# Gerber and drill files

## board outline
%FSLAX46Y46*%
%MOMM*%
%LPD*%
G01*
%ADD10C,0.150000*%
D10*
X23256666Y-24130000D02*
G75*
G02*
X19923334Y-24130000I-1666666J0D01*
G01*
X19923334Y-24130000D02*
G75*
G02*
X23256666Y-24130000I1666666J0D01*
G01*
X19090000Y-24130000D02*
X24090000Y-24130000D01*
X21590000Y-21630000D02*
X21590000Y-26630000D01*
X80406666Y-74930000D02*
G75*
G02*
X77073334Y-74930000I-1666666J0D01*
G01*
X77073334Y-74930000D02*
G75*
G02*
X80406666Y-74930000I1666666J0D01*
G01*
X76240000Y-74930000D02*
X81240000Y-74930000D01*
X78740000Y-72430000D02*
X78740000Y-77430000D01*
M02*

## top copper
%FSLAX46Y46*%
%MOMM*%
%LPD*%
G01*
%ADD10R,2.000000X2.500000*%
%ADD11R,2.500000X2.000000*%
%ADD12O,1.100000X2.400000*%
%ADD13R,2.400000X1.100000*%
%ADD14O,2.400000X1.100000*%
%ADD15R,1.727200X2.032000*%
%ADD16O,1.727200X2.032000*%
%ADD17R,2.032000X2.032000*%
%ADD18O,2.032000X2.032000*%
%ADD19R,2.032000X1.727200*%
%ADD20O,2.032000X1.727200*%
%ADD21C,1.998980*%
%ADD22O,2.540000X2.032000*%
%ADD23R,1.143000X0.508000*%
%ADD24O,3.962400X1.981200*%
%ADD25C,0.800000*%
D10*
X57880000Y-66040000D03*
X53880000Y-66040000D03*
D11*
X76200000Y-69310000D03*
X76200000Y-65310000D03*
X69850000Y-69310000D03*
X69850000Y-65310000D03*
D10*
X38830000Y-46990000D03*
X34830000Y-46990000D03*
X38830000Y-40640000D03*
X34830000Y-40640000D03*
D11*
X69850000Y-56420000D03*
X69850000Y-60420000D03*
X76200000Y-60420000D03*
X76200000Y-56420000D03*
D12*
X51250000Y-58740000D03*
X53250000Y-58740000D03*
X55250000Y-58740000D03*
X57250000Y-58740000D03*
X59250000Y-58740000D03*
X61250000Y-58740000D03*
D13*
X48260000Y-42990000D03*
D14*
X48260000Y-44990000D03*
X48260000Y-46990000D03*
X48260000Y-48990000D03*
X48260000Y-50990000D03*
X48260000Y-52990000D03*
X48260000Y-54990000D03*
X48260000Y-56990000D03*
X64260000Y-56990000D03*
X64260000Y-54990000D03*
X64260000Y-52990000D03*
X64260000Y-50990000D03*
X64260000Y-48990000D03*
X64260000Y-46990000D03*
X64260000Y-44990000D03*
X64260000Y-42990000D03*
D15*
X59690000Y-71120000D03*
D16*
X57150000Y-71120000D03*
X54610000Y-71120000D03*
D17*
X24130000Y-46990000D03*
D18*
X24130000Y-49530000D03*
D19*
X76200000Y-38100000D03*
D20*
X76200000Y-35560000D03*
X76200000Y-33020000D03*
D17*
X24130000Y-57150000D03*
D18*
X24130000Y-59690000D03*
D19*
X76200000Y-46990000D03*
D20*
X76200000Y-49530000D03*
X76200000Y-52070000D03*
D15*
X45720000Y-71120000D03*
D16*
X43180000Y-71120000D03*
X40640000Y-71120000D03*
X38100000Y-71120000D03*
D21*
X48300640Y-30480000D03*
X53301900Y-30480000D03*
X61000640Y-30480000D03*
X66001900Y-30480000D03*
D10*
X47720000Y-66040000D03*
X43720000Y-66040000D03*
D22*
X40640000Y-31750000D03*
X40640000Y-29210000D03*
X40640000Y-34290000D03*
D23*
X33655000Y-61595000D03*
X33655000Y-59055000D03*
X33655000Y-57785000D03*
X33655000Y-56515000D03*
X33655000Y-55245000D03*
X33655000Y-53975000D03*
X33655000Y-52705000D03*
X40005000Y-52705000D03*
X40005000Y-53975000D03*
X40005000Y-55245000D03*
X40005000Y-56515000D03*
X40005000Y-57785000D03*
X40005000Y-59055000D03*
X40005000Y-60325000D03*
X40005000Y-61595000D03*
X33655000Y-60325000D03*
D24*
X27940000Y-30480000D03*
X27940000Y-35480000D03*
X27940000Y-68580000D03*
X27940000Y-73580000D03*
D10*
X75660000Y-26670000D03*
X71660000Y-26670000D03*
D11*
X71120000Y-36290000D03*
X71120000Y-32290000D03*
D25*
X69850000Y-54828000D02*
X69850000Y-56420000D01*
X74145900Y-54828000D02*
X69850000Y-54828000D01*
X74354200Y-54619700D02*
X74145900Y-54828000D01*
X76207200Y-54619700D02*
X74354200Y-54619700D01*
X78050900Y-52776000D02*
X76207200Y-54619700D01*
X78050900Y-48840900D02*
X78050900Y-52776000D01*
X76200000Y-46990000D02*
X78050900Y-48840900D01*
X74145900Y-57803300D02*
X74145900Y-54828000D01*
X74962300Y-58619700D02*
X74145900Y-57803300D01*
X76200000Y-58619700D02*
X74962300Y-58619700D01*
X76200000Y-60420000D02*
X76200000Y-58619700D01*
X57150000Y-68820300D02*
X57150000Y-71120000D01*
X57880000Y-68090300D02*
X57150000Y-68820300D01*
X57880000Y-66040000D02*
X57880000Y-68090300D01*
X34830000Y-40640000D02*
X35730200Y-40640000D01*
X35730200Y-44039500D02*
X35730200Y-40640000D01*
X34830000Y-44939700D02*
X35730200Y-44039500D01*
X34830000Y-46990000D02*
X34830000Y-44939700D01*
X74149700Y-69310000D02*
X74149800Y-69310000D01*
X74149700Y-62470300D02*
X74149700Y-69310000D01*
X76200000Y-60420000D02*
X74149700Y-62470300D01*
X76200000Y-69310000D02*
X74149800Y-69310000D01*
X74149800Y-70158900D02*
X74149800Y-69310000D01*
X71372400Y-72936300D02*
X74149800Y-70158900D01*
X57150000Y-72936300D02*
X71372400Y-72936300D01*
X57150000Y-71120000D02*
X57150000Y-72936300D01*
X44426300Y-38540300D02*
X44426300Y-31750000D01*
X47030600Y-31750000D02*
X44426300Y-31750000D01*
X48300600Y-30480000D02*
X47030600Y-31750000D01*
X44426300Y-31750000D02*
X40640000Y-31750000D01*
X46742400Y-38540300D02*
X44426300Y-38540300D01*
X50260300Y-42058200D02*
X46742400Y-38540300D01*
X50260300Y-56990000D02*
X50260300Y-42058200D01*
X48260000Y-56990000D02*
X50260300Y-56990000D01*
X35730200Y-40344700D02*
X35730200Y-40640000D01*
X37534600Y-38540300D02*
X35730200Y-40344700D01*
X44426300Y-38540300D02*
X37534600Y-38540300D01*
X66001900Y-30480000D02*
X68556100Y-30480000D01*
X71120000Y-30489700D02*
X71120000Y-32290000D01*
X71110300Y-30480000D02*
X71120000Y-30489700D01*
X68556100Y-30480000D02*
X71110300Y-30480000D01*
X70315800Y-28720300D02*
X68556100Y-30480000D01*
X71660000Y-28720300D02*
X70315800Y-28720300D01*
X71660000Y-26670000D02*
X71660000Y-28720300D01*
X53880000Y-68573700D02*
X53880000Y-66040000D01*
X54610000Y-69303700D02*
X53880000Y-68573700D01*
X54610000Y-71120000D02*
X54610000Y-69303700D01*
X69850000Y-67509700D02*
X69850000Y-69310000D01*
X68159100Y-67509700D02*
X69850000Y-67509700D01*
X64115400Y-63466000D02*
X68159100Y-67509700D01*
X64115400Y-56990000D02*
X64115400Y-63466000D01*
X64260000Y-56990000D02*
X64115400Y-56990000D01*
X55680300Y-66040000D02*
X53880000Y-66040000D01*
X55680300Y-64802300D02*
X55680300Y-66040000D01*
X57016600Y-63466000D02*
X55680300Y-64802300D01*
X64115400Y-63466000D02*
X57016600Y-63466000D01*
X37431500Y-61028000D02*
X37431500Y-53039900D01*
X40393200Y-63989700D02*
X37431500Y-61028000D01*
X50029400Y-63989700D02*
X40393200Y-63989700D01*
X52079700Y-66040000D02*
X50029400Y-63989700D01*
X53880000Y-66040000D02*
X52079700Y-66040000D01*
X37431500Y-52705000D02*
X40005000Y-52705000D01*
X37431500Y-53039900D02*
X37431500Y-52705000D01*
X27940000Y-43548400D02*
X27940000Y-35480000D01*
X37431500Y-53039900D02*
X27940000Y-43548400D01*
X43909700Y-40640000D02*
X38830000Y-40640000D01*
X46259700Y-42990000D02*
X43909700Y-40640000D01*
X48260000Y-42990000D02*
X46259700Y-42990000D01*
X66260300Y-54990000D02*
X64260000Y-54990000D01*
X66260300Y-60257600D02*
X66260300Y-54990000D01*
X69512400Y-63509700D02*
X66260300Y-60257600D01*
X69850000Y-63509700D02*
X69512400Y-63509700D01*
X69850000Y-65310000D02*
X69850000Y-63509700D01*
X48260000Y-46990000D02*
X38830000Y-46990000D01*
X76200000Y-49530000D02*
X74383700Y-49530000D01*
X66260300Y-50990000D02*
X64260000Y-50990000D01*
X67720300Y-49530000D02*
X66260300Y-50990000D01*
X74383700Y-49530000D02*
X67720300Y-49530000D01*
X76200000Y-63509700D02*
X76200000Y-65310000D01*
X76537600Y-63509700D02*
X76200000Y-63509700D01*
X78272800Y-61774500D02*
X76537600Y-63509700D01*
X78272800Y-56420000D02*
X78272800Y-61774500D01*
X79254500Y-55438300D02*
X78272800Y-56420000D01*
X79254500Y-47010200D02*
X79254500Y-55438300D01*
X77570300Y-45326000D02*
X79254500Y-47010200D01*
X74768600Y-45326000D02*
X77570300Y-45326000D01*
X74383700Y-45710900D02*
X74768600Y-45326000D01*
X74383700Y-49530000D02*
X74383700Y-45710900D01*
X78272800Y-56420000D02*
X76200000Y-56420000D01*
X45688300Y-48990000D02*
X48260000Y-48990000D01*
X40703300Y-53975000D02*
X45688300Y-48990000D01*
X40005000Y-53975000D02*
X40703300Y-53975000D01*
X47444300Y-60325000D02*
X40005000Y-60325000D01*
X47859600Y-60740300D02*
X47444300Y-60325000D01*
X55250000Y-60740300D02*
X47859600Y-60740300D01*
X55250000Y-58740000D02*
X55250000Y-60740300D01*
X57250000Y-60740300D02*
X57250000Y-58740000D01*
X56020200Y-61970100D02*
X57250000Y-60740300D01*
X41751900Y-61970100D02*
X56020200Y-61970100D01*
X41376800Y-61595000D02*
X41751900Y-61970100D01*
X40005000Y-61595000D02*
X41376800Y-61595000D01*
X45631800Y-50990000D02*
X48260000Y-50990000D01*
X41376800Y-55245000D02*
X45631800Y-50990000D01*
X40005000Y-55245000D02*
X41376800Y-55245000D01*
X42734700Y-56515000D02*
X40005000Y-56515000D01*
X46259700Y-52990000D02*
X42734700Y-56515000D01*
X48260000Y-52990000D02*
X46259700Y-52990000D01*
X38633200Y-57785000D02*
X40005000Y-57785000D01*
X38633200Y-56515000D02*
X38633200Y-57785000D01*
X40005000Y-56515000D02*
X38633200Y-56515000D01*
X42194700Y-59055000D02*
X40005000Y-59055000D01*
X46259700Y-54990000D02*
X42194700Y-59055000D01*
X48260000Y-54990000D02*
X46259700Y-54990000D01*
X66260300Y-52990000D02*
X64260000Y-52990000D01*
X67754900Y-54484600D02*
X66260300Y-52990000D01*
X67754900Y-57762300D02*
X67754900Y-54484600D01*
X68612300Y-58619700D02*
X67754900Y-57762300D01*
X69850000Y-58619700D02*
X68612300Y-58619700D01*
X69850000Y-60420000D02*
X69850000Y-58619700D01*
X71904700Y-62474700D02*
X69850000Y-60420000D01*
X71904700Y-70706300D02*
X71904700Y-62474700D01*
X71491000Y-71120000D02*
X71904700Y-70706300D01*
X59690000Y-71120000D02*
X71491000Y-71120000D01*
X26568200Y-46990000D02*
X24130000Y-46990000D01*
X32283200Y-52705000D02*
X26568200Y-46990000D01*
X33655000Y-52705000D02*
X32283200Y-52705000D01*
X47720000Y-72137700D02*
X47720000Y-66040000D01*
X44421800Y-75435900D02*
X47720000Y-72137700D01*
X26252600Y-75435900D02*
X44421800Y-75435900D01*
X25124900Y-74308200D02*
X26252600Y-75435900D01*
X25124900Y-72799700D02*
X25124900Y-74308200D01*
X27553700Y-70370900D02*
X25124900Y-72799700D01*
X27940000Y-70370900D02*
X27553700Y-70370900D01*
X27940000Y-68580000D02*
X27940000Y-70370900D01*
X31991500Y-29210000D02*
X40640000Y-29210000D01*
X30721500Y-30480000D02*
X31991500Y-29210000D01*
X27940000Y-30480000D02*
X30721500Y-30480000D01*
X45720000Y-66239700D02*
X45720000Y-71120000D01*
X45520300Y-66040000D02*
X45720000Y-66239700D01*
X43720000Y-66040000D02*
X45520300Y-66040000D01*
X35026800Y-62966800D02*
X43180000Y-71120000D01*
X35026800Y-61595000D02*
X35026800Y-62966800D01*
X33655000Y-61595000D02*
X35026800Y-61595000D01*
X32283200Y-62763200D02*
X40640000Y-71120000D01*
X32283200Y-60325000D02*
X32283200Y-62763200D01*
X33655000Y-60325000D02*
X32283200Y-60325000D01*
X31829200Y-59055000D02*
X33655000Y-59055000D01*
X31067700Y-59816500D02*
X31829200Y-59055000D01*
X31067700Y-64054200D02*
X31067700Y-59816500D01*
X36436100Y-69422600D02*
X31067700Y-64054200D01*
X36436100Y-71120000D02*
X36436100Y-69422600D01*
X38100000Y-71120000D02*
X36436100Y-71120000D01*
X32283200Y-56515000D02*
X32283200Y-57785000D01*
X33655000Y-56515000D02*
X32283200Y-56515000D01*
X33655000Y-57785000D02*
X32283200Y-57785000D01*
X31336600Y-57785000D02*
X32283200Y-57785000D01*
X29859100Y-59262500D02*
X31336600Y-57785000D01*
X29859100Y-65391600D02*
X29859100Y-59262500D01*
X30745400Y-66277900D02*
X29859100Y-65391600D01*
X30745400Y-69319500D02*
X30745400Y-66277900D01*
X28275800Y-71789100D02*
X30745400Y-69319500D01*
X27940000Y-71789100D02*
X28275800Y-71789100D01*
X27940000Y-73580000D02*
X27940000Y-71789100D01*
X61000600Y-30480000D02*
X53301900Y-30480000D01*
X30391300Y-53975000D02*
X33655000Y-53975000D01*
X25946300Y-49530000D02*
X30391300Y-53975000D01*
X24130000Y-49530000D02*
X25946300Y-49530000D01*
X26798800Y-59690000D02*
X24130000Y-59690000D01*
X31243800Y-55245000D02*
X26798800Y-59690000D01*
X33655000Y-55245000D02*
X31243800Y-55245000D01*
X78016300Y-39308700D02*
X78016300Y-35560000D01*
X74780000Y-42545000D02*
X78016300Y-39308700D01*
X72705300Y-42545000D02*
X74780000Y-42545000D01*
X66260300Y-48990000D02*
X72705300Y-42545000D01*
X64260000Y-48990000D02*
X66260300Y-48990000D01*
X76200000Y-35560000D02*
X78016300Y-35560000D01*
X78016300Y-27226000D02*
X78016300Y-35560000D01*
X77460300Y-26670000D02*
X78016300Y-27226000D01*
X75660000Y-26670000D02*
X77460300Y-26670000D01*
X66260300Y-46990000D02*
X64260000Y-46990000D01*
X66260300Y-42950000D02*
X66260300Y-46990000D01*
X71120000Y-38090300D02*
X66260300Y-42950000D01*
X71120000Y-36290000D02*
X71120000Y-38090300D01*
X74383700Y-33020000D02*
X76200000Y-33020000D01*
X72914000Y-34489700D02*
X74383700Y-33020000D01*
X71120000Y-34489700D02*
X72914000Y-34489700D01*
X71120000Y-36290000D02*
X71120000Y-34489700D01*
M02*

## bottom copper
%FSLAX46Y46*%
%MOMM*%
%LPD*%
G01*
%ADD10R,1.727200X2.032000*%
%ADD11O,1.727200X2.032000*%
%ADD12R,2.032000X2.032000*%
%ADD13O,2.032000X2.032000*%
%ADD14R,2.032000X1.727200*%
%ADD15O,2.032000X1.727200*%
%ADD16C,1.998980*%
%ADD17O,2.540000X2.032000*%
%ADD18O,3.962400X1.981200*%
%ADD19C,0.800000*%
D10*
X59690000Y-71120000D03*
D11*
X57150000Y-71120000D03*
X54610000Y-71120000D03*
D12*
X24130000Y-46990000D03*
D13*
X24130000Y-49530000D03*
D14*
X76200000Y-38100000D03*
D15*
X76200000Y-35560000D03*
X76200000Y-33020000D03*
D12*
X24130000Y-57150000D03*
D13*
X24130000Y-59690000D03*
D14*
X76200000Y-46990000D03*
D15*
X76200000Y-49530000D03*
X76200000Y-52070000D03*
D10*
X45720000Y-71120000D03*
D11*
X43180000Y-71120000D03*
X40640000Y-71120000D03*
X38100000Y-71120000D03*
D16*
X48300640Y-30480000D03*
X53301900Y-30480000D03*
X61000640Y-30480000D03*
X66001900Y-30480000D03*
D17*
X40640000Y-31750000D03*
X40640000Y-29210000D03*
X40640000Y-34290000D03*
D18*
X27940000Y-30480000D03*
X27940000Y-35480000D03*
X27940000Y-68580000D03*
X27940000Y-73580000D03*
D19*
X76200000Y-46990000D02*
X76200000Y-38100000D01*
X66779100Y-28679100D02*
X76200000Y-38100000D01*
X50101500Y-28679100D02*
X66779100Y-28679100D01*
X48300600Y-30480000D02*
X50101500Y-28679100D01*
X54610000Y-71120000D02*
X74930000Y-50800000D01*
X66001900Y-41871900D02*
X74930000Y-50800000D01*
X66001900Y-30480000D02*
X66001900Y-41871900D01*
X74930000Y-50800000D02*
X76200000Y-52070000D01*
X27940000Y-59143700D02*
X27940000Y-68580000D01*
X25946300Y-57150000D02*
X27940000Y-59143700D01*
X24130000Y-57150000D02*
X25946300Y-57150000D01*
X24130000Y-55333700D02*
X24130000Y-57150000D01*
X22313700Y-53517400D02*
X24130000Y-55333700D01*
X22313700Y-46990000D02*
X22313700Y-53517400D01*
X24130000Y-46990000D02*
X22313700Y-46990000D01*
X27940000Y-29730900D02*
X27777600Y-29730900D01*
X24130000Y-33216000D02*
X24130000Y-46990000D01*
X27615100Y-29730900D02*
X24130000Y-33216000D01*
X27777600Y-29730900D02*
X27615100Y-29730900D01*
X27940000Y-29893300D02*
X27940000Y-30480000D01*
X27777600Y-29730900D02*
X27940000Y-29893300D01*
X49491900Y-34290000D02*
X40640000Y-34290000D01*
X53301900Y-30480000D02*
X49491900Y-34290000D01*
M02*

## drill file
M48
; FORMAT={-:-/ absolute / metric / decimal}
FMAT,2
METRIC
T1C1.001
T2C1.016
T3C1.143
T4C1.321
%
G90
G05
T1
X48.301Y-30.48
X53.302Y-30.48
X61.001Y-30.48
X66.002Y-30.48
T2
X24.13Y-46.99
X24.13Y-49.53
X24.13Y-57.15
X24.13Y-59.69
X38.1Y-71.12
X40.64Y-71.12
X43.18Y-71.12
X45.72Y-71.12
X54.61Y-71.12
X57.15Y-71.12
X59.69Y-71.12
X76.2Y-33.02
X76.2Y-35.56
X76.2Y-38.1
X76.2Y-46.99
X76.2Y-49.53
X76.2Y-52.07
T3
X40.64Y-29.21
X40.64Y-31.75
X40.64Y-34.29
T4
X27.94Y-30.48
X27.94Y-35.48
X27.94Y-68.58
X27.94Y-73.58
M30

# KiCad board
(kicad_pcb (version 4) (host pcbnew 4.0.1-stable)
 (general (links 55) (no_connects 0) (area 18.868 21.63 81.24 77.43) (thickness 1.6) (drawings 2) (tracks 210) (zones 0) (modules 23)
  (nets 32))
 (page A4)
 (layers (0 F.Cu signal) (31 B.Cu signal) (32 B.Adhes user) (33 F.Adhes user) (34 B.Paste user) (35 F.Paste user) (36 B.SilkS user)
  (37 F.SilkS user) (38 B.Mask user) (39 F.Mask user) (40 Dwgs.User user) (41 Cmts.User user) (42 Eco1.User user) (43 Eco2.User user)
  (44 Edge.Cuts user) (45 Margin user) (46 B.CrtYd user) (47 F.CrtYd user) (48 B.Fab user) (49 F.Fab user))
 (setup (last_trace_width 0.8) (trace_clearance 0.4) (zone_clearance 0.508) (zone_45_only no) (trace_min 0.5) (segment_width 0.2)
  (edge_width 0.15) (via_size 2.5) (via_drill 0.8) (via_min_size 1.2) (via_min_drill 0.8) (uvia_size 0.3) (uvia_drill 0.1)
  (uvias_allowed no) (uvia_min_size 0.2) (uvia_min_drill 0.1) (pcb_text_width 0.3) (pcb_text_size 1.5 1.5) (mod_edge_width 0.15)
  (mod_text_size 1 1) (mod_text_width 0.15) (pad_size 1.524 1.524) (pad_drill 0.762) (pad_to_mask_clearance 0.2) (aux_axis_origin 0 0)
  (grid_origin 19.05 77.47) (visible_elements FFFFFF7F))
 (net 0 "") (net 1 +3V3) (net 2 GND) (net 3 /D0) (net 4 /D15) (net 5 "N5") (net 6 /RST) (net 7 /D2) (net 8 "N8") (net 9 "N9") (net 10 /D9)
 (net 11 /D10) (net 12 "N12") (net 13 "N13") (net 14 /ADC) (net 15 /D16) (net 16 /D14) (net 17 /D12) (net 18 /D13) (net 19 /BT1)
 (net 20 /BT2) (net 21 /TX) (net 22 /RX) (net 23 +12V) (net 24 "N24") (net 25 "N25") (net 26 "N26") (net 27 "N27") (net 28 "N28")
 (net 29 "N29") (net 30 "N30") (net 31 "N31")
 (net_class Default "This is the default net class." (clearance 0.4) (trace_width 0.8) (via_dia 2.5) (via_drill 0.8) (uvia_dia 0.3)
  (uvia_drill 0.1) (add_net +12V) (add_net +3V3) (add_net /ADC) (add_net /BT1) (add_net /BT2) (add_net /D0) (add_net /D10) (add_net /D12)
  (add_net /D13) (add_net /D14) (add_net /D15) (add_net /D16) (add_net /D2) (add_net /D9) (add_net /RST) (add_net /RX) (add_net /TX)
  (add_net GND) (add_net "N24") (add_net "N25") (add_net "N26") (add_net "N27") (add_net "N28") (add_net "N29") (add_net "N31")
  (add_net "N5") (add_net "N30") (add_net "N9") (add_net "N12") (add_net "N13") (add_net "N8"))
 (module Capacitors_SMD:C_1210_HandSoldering (layer F.Cu) (at 55.88 66.04 180)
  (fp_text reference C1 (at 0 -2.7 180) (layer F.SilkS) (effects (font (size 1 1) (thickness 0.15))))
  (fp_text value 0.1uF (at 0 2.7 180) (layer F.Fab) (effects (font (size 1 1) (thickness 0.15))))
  (pad 1 smd rect (at -2 0 180) (size 2 2.5) (layers F.Cu F.Paste F.Mask) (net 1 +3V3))
  (pad 2 smd rect (at 2 0 180) (size 2 2.5) (layers F.Cu F.Paste F.Mask) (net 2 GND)))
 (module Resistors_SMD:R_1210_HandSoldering (layer F.Cu) (at 76.2 67.31 90)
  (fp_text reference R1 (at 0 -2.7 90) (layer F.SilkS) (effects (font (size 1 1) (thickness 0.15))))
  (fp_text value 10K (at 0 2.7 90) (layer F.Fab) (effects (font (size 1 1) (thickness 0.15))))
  (pad 1 smd rect (at -2 0 90) (size 2 2.5) (layers F.Cu F.Paste F.Mask) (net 1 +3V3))
  (pad 2 smd rect (at 2 0 90) (size 2 2.5) (layers F.Cu F.Paste F.Mask) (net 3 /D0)))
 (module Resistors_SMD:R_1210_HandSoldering (layer F.Cu) (at 69.85 67.31 90)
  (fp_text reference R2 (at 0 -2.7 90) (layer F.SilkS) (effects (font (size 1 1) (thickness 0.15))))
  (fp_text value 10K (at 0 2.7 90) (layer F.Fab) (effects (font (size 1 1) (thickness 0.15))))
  (pad 1 smd rect (at -2 0 90) (size 2 2.5) (layers F.Cu F.Paste F.Mask) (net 2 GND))
  (pad 2 smd rect (at 2 0 90) (size 2 2.5) (layers F.Cu F.Paste F.Mask) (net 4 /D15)))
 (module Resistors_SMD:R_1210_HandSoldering (layer F.Cu) (at 36.83 46.99 180)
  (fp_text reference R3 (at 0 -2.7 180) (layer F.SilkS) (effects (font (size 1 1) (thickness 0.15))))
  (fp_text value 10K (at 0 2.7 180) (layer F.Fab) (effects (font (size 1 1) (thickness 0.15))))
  (pad 1 smd rect (at -2 0 180) (size 2 2.5) (layers F.Cu F.Paste F.Mask) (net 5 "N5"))
  (pad 2 smd rect (at 2 0 180) (size 2 2.5) (layers F.Cu F.Paste F.Mask) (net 1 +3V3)))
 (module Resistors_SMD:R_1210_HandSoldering (layer F.Cu) (at 36.83 40.64 180)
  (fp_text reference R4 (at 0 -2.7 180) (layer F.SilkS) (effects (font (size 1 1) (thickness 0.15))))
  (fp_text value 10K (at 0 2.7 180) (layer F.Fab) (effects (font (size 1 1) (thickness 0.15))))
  (pad 1 smd rect (at -2 0 180) (size 2 2.5) (layers F.Cu F.Paste F.Mask) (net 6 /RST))
  (pad 2 smd rect (at 2 0 180) (size 2 2.5) (layers F.Cu F.Paste F.Mask) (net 1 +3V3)))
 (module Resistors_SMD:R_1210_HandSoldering (layer F.Cu) (at 69.85 58.42 270)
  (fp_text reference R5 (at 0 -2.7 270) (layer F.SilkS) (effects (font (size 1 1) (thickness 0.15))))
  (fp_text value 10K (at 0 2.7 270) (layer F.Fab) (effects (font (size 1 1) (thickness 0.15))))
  (pad 1 smd rect (at -2 0 270) (size 2 2.5) (layers F.Cu F.Paste F.Mask) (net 1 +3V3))
  (pad 2 smd rect (at 2 0 270) (size 2 2.5) (layers F.Cu F.Paste F.Mask) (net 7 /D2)))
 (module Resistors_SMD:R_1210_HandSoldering (layer F.Cu) (at 76.2 58.42 90)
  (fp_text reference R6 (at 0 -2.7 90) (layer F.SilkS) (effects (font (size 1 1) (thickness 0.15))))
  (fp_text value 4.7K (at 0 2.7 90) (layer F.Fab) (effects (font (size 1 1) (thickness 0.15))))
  (pad 1 smd rect (at -2 0 90) (size 2 2.5) (layers F.Cu F.Paste F.Mask) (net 1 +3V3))
  (pad 2 smd rect (at 2 0 90) (size 2 2.5) (layers F.Cu F.Paste F.Mask) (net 3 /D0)))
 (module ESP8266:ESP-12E (layer F.Cu) (at 48.26 42.99)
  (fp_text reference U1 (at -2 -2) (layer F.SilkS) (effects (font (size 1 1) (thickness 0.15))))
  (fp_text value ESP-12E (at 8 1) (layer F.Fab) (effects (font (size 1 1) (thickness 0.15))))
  (pad 9 smd oval (at 2.99 15.75 90) (size 2.4 1.1) (layers F.Cu F.Paste F.Mask) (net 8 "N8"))
  (pad 10 smd oval (at 4.99 15.75 90) (size 2.4 1.1) (layers F.Cu F.Paste F.Mask) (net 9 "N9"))
  (pad 11 smd oval (at 6.99 15.75 90) (size 2.4 1.1) (layers F.Cu F.Paste F.Mask) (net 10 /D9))
  (pad 12 smd oval (at 8.99 15.75 90) (size 2.4 1.1) (layers F.Cu F.Paste F.Mask) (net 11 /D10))
  (pad 13 smd oval (at 10.99 15.75 90) (size 2.4 1.1) (layers F.Cu F.Paste F.Mask) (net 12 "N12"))
  (pad 14 smd oval (at 12.99 15.75 90) (size 2.4 1.1) (layers F.Cu F.Paste F.Mask) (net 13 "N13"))
  (pad 1 smd rect (at 0 0) (size 2.4 1.1) (layers F.Cu F.Paste F.Mask) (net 6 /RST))
  (pad 2 smd oval (at 0 2) (size 2.4 1.1) (layers F.Cu F.Paste F.Mask) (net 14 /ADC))
  (pad 3 smd oval (at 0 4) (size 2.4 1.1) (layers F.Cu F.Paste F.Mask) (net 5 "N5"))
  (pad 4 smd oval (at 0 6) (size 2.4 1.1) (layers F.Cu F.Paste F.Mask) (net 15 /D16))
  (pad 5 smd oval (at 0 8) (size 2.4 1.1) (layers F.Cu F.Paste F.Mask) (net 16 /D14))
  (pad 6 smd oval (at 0 10) (size 2.4 1.1) (layers F.Cu F.Paste F.Mask) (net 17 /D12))
  (pad 7 smd oval (at 0 12) (size 2.4 1.1) (layers F.Cu F.Paste F.Mask) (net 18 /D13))
  (pad 8 smd oval (at 0 14) (size 2.4 1.1) (layers F.Cu F.Paste F.Mask) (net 1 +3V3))
  (pad 15 smd oval (at 16 14) (size 2.4 1.1) (layers F.Cu F.Paste F.Mask) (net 2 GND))
  (pad 16 smd oval (at 16 12) (size 2.4 1.1) (layers F.Cu F.Paste F.Mask) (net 4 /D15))
  (pad 17 smd oval (at 16 10) (size 2.4 1.1) (layers F.Cu F.Paste F.Mask) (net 7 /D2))
  (pad 18 smd oval (at 16 8) (size 2.4 1.1) (layers F.Cu F.Paste F.Mask) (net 3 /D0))
  (pad 19 smd oval (at 16 6) (size 2.4 1.1) (layers F.Cu F.Paste F.Mask) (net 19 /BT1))
  (pad 20 smd oval (at 16 4) (size 2.4 1.1) (layers F.Cu F.Paste F.Mask) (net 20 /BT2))
  (pad 21 smd oval (at 16 2) (size 2.4 1.1) (layers F.Cu F.Paste F.Mask) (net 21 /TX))
  (pad 22 smd oval (at 16 0) (size 2.4 1.1) (layers F.Cu F.Paste F.Mask) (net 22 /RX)))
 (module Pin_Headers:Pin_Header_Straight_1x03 (layer F.Cu) (at 59.69 71.12 270)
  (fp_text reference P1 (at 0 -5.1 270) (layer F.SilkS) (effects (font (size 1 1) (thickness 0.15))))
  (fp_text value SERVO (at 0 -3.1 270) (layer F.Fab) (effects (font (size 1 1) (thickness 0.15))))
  (pad 1 thru_hole rect (at 0 0 270) (size 2.032 1.7272) (drill 1.016) (layers *.Cu *.Mask F.SilkS) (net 7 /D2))
  (pad 2 thru_hole oval (at 0 2.54 270) (size 2.032 1.7272) (drill 1.016) (layers *.Cu *.Mask F.SilkS) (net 1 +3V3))
  (pad 3 thru_hole oval (at 0 5.08 270) (size 2.032 1.7272) (drill 1.016) (layers *.Cu *.Mask F.SilkS) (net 2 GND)))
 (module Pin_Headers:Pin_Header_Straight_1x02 (layer F.Cu) (at 24.13 46.99)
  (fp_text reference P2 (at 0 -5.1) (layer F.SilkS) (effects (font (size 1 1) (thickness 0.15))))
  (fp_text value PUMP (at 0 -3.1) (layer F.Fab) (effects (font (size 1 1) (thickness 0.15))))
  (pad 1 thru_hole rect (at 0 0) (size 2.032 2.032) (drill 1.016) (layers *.Cu *.Mask F.SilkS) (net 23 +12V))
  (pad 2 thru_hole oval (at 0 2.54) (size 2.032 2.032) (drill 1.016) (layers *.Cu *.Mask F.SilkS) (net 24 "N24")))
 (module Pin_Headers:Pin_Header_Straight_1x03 (layer F.Cu) (at 76.2 38.1 180)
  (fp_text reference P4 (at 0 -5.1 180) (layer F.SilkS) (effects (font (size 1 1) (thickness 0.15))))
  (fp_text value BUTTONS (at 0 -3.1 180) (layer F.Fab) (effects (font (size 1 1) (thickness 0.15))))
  (pad 1 thru_hole rect (at 0 0 180) (size 2.032 1.7272) (drill 1.016) (layers *.Cu *.Mask F.SilkS) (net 1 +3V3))
  (pad 2 thru_hole oval (at 0 2.54 180) (size 2.032 1.7272) (drill 1.016) (layers *.Cu *.Mask F.SilkS) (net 19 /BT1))
  (pad 3 thru_hole oval (at 0 5.08 180) (size 2.032 1.7272) (drill 1.016) (layers *.Cu *.Mask F.SilkS) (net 20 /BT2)))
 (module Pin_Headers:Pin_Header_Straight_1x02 (layer F.Cu) (at 24.13 57.15)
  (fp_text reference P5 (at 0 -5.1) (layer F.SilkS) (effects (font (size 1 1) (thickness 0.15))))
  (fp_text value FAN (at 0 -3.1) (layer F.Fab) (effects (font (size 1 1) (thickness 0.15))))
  (pad 1 thru_hole rect (at 0 0) (size 2.032 2.032) (drill 1.016) (layers *.Cu *.Mask F.SilkS) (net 23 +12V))
  (pad 2 thru_hole oval (at 0 2.54) (size 2.032 2.032) (drill 1.016) (layers *.Cu *.Mask F.SilkS) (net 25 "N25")))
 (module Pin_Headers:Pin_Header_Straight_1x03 (layer F.Cu) (at 76.2 46.99)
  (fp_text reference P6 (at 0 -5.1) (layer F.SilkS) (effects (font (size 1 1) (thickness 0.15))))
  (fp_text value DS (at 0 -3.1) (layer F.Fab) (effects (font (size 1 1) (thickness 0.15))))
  (pad 1 thru_hole rect (at 0 0) (size 2.032 1.7272) (drill 1.016) (layers *.Cu *.Mask F.SilkS) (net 1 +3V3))
  (pad 2 thru_hole oval (at 0 2.54) (size 2.032 1.7272) (drill 1.016) (layers *.Cu *.Mask F.SilkS) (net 3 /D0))
  (pad 3 thru_hole oval (at 0 5.08) (size 2.032 1.7272) (drill 1.016) (layers *.Cu *.Mask F.SilkS) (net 2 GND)))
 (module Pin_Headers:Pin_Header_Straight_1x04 (layer F.Cu) (at 45.72 71.12 270)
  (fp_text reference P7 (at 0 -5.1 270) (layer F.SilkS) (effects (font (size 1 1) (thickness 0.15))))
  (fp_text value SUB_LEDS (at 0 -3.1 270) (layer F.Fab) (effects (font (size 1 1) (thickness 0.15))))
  (pad 1 thru_hole rect (at 0 0 270) (size 2.032 1.7272) (drill 1.016) (layers *.Cu *.Mask F.SilkS) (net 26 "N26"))
  (pad 2 thru_hole oval (at 0 2.54 270) (size 2.032 1.7272) (drill 1.016) (layers *.Cu *.Mask F.SilkS) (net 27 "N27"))
  (pad 3 thru_hole oval (at 0 5.08 270) (size 2.032 1.7272) (drill 1.016) (layers *.Cu *.Mask F.SilkS) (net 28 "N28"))
  (pad 4 thru_hole oval (at 0 7.62 270) (size 2.032 1.7272) (drill 1.016) (layers *.Cu *.Mask F.SilkS) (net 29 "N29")))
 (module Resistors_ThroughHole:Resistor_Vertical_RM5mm (layer F.Cu) (at 50.8 30.48)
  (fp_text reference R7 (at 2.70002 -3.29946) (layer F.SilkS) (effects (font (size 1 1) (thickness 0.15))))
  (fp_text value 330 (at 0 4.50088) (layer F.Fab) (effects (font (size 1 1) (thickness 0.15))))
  (pad 1 thru_hole circle (at -2.49936 0) (size 1.99898 1.99898) (drill 1.00076) (layers *.Cu *.SilkS *.Mask) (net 1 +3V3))
  (pad 2 thru_hole circle (at 2.5019 0) (size 1.99898 1.99898) (drill 1.00076) (layers *.Cu *.SilkS *.Mask) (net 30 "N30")))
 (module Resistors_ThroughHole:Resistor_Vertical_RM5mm (layer F.Cu) (at 63.5 30.48)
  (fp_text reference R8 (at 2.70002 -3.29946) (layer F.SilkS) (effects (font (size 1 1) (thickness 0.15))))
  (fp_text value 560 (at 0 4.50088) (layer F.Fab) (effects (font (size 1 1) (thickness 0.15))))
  (pad 1 thru_hole circle (at -2.49936 0) (size 1.99898 1.99898) (drill 1.00076) (layers *.Cu *.SilkS *.Mask) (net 30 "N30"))
  (pad 2 thru_hole circle (at 2.5019 0) (size 1.99898 1.99898) (drill 1.00076) (layers *.Cu *.SilkS *.Mask) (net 2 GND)))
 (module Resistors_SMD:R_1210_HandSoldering (layer F.Cu) (at 45.72 66.04 180)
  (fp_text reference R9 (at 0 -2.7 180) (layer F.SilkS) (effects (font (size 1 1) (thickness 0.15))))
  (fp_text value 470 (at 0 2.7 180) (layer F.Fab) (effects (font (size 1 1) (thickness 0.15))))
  (pad 1 smd rect (at -2 0 180) (size 2 2.5) (layers F.Cu F.Paste F.Mask) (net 23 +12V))
  (pad 2 smd rect (at 2 0 180) (size 2 2.5) (layers F.Cu F.Paste F.Mask) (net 26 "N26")))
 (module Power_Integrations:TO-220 (layer F.Cu) (at 40.64 31.75 90)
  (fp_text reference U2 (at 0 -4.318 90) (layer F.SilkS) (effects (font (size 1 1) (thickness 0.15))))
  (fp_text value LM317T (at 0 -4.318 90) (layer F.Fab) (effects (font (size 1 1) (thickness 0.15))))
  (pad 2 thru_hole oval (at 0 0 90) (size 2.032 2.54) (drill 1.143) (layers *.Cu *.Mask F.SilkS) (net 1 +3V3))
  (pad 3 thru_hole oval (at 2.54 0 90) (size 2.032 2.54) (drill 1.143) (layers *.Cu *.Mask F.SilkS) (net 23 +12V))
  (pad 1 thru_hole oval (at -2.54 0 90) (size 2.032 2.54) (drill 1.143) (layers *.Cu *.Mask F.SilkS) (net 30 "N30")))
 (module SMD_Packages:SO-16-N (layer F.Cu) (at 36.83 57.15 90)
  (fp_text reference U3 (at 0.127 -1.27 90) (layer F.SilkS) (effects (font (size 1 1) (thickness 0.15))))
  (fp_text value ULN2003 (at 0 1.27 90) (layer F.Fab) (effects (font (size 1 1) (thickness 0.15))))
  (pad 16 smd rect (at -4.445 -3.175 90) (size 0.508 1.143) (layers F.Cu F.Paste F.Mask) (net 27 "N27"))
  (pad 14 smd rect (at -1.905 -3.175 90) (size 0.508 1.143) (layers F.Cu F.Paste F.Mask) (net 29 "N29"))
  (pad 13 smd rect (at -0.635 -3.175 90) (size 0.508 1.143) (layers F.Cu F.Paste F.Mask) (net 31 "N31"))
  (pad 12 smd rect (at 0.635 -3.175 90) (size 0.508 1.143) (layers F.Cu F.Paste F.Mask) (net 31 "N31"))
  (pad 11 smd rect (at 1.905 -3.175 90) (size 0.508 1.143) (layers F.Cu F.Paste F.Mask) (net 25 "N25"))
  (pad 10 smd rect (at 3.175 -3.175 90) (size 0.508 1.143) (layers F.Cu F.Paste F.Mask) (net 24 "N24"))
  (pad 9 smd rect (at 4.445 -3.175 90) (size 0.508 1.143) (layers F.Cu F.Paste F.Mask) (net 23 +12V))
  (pad 8 smd rect (at 4.445 3.175 90) (size 0.508 1.143) (layers F.Cu F.Paste F.Mask) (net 2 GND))
  (pad 7 smd rect (at 3.175 3.175 90) (size 0.508 1.143) (layers F.Cu F.Paste F.Mask) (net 15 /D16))
  (pad 6 smd rect (at 1.905 3.175 90) (size 0.508 1.143) (layers F.Cu F.Paste F.Mask) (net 16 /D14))
  (pad 5 smd rect (at 0.635 3.175 90) (size 0.508 1.143) (layers F.Cu F.Paste F.Mask) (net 17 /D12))
  (pad 4 smd rect (at -0.635 3.175 90) (size 0.508 1.143) (layers F.Cu F.Paste F.Mask) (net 17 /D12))
  (pad 3 smd rect (at -1.905 3.175 90) (size 0.508 1.143) (layers F.Cu F.Paste F.Mask) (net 18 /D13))
  (pad 2 smd rect (at -3.175 3.175 90) (size 0.508 1.143) (layers F.Cu F.Paste F.Mask) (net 10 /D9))
  (pad 1 smd rect (at -4.445 3.175 90) (size 0.508 1.143) (layers F.Cu F.Paste F.Mask) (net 11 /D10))
  (pad 15 smd rect (at -3.175 -3.175 90) (size 0.508 1.143) (layers F.Cu F.Paste F.Mask) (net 28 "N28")))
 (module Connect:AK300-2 (layer F.Cu) (at 27.94 30.48 270)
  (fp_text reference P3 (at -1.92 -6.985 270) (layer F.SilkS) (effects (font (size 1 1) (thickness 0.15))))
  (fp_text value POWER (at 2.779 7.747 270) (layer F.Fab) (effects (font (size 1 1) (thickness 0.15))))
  (pad 1 thru_hole oval (at 0 0 270) (size 1.9812 3.9624) (drill 1.3208) (layers *.Cu F.Paste F.SilkS F.Mask) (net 23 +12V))
  (pad 2 thru_hole oval (at 5 0 270) (size 1.9812 3.9624) (drill 1.3208) (layers *.Cu F.Paste F.SilkS F.Mask) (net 2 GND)))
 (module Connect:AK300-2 (layer F.Cu) (at 27.94 68.58 270)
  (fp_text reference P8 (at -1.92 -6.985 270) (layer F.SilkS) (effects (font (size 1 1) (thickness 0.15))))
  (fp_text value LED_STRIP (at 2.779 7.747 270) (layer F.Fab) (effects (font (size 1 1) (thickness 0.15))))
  (pad 1 thru_hole oval (at 0 0 270) (size 1.9812 3.9624) (drill 1.3208) (layers *.Cu F.Paste F.SilkS F.Mask) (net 23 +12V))
  (pad 2 thru_hole oval (at 5 0 270) (size 1.9812 3.9624) (drill 1.3208) (layers *.Cu F.Paste F.SilkS F.Mask) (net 31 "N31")))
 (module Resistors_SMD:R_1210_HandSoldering (layer F.Cu) (at 73.66 26.67 180)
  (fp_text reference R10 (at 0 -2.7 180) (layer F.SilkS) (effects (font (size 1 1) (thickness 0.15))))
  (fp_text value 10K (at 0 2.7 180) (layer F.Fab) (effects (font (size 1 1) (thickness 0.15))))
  (pad 1 smd rect (at -2 0 180) (size 2 2.5) (layers F.Cu F.Paste F.Mask) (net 19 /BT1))
  (pad 2 smd rect (at 2 0 180) (size 2 2.5) (layers F.Cu F.Paste F.Mask) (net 2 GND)))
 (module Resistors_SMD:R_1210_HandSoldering (layer F.Cu) (at 71.12 34.29 90)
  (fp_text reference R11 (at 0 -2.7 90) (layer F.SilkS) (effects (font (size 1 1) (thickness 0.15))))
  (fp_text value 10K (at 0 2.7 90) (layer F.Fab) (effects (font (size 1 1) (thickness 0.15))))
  (pad 1 smd rect (at -2 0 90) (size 2 2.5) (layers F.Cu F.Paste F.Mask) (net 20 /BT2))
  (pad 2 smd rect (at 2 0 90) (size 2 2.5) (layers F.Cu F.Paste F.Mask) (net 2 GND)))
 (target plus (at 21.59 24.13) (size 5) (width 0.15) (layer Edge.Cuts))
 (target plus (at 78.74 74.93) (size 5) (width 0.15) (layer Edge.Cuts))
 (segment (start 76.2 46.99) (end 76.2 38.1) (width 0.8) (layer B.Cu) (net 1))
 (segment (start 69.85 54.828) (end 69.85 56.42) (width 0.8) (layer F.Cu) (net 1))
 (segment (start 74.1459 54.828) (end 69.85 54.828) (width 0.8) (layer F.Cu) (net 1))
 (segment (start 74.3542 54.6197) (end 74.1459 54.828) (width 0.8) (layer F.Cu) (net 1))
 (segment (start 76.2072 54.6197) (end 74.3542 54.6197) (width 0.8) (layer F.Cu) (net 1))
 (segment (start 78.0509 52.776) (end 76.2072 54.6197) (width 0.8) (layer F.Cu) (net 1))
 (segment (start 78.0509 48.8409) (end 78.0509 52.776) (width 0.8) (layer F.Cu) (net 1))
 (segment (start 76.2 46.99) (end 78.0509 48.8409) (width 0.8) (layer F.Cu) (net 1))
 (segment (start 74.1459 57.8033) (end 74.1459 54.828) (width 0.8) (layer F.Cu) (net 1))
 (segment (start 74.9623 58.6197) (end 74.1459 57.8033) (width 0.8) (layer F.Cu) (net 1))
 (segment (start 76.2 58.6197) (end 74.9623 58.6197) (width 0.8) (layer F.Cu) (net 1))
 (segment (start 76.2 60.42) (end 76.2 58.6197) (width 0.8) (layer F.Cu) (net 1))
 (segment (start 66.7791 28.6791) (end 76.2 38.1) (width 0.8) (layer B.Cu) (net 1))
 (segment (start 50.1015 28.6791) (end 66.7791 28.6791) (width 0.8) (layer B.Cu) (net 1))
 (segment (start 48.3006 30.48) (end 50.1015 28.6791) (width 0.8) (layer B.Cu) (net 1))
 (segment (start 57.15 68.8203) (end 57.15 71.12) (width 0.8) (layer F.Cu) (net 1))
 (segment (start 57.88 68.0903) (end 57.15 68.8203) (width 0.8) (layer F.Cu) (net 1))
 (segment (start 57.88 66.04) (end 57.88 68.0903) (width 0.8) (layer F.Cu) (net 1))
 (segment (start 34.83 40.64) (end 35.7302 40.64) (width 0.8) (layer F.Cu) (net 1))
 (segment (start 35.7302 44.0395) (end 35.7302 40.64) (width 0.8) (layer F.Cu) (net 1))
 (segment (start 34.83 44.9397) (end 35.7302 44.0395) (width 0.8) (layer F.Cu) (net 1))
 (segment (start 34.83 46.99) (end 34.83 44.9397) (width 0.8) (layer F.Cu) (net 1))
 (segment (start 74.1497 69.31) (end 74.1498 69.31) (width 0.8) (layer F.Cu) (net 1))
 (segment (start 74.1497 62.4703) (end 74.1497 69.31) (width 0.8) (layer F.Cu) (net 1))
 (segment (start 76.2 60.42) (end 74.1497 62.4703) (width 0.8) (layer F.Cu) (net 1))
 (segment (start 76.2 69.31) (end 74.1498 69.31) (width 0.8) (layer F.Cu) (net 1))
 (segment (start 74.1498 70.1589) (end 74.1498 69.31) (width 0.8) (layer F.Cu) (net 1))
 (segment (start 71.3724 72.9363) (end 74.1498 70.1589) (width 0.8) (layer F.Cu) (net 1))
 (segment (start 57.15 72.9363) (end 71.3724 72.9363) (width 0.8) (layer F.Cu) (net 1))
 (segment (start 57.15 71.12) (end 57.15 72.9363) (width 0.8) (layer F.Cu) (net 1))
 (segment (start 44.4263 38.5403) (end 44.4263 31.75) (width 0.8) (layer F.Cu) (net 1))
 (segment (start 47.0306 31.75) (end 44.4263 31.75) (width 0.8) (layer F.Cu) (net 1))
 (segment (start 48.3006 30.48) (end 47.0306 31.75) (width 0.8) (layer F.Cu) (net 1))
 (segment (start 44.4263 31.75) (end 40.64 31.75) (width 0.8) (layer F.Cu) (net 1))
 (segment (start 46.7424 38.5403) (end 44.4263 38.5403) (width 0.8) (layer F.Cu) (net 1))
 (segment (start 50.2603 42.0582) (end 46.7424 38.5403) (width 0.8) (layer F.Cu) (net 1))
 (segment (start 50.2603 56.99) (end 50.2603 42.0582) (width 0.8) (layer F.Cu) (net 1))
 (segment (start 48.26 56.99) (end 50.2603 56.99) (width 0.8) (layer F.Cu) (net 1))
 (segment (start 35.7302 40.3447) (end 35.7302 40.64) (width 0.8) (layer F.Cu) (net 1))
 (segment (start 37.5346 38.5403) (end 35.7302 40.3447) (width 0.8) (layer F.Cu) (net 1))
 (segment (start 44.4263 38.5403) (end 37.5346 38.5403) (width 0.8) (layer F.Cu) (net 1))
 (segment (start 66.0019 30.48) (end 68.5561 30.48) (width 0.8) (layer F.Cu) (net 2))
 (segment (start 71.12 30.4897) (end 71.12 32.29) (width 0.8) (layer F.Cu) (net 2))
 (segment (start 71.1103 30.48) (end 71.12 30.4897) (width 0.8) (layer F.Cu) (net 2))
 (segment (start 68.5561 30.48) (end 71.1103 30.48) (width 0.8) (layer F.Cu) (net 2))
 (segment (start 70.3158 28.7203) (end 68.5561 30.48) (width 0.8) (layer F.Cu) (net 2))
 (segment (start 71.66 28.7203) (end 70.3158 28.7203) (width 0.8) (layer F.Cu) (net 2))
 (segment (start 71.66 26.67) (end 71.66 28.7203) (width 0.8) (layer F.Cu) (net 2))
 (segment (start 53.88 68.5737) (end 53.88 66.04) (width 0.8) (layer F.Cu) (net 2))
 (segment (start 54.61 69.3037) (end 53.88 68.5737) (width 0.8) (layer F.Cu) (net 2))
 (segment (start 54.61 71.12) (end 54.61 69.3037) (width 0.8) (layer F.Cu) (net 2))
 (segment (start 69.85 67.5097) (end 69.85 69.31) (width 0.8) (layer F.Cu) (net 2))
 (segment (start 68.1591 67.5097) (end 69.85 67.5097) (width 0.8) (layer F.Cu) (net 2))
 (segment (start 64.1154 63.466) (end 68.1591 67.5097) (width 0.8) (layer F.Cu) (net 2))
 (segment (start 64.1154 56.99) (end 64.1154 63.466) (width 0.8) (layer F.Cu) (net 2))
 (segment (start 64.26 56.99) (end 64.1154 56.99) (width 0.8) (layer F.Cu) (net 2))
 (segment (start 55.6803 66.04) (end 53.88 66.04) (width 0.8) (layer F.Cu) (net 2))
 (segment (start 55.6803 64.8023) (end 55.6803 66.04) (width 0.8) (layer F.Cu) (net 2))
 (segment (start 57.0166 63.466) (end 55.6803 64.8023) (width 0.8) (layer F.Cu) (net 2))
 (segment (start 64.1154 63.466) (end 57.0166 63.466) (width 0.8) (layer F.Cu) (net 2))
 (segment (start 54.61 71.12) (end 74.93 50.8) (width 0.8) (layer B.Cu) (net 2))
 (segment (start 66.0019 41.8719) (end 74.93 50.8) (width 0.8) (layer B.Cu) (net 2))
 (segment (start 66.0019 30.48) (end 66.0019 41.8719) (width 0.8) (layer B.Cu) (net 2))
 (segment (start 74.93 50.8) (end 76.2 52.07) (width 0.8) (layer B.Cu) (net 2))
 (segment (start 37.4315 61.028) (end 37.4315 53.0399) (width 0.8) (layer F.Cu) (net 2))
 (segment (start 40.3932 63.9897) (end 37.4315 61.028) (width 0.8) (layer F.Cu) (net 2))
 (segment (start 50.0294 63.9897) (end 40.3932 63.9897) (width 0.8) (layer F.Cu) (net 2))
 (segment (start 52.0797 66.04) (end 50.0294 63.9897) (width 0.8) (layer F.Cu) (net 2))
 (segment (start 53.88 66.04) (end 52.0797 66.04) (width 0.8) (layer F.Cu) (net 2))
 (segment (start 37.4315 52.705) (end 40.005 52.705) (width 0.8) (layer F.Cu) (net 2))
 (segment (start 37.4315 53.0399) (end 37.4315 52.705) (width 0.8) (layer F.Cu) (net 2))
 (segment (start 27.94 43.5484) (end 27.94 35.48) (width 0.8) (layer F.Cu) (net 2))
 (segment (start 37.4315 53.0399) (end 27.94 43.5484) (width 0.8) (layer F.Cu) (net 2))
 (segment (start 43.9097 40.64) (end 38.83 40.64) (width 0.8) (layer F.Cu) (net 6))
 (segment (start 46.2597 42.99) (end 43.9097 40.64) (width 0.8) (layer F.Cu) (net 6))
 (segment (start 48.26 42.99) (end 46.2597 42.99) (width 0.8) (layer F.Cu) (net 6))
 (segment (start 66.2603 54.99) (end 64.26 54.99) (width 0.8) (layer F.Cu) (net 4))
 (segment (start 66.2603 60.2576) (end 66.2603 54.99) (width 0.8) (layer F.Cu) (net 4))
 (segment (start 69.5124 63.5097) (end 66.2603 60.2576) (width 0.8) (layer F.Cu) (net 4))
 (segment (start 69.85 63.5097) (end 69.5124 63.5097) (width 0.8) (layer F.Cu) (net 4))
 (segment (start 69.85 65.31) (end 69.85 63.5097) (width 0.8) (layer F.Cu) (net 4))
 (segment (start 48.26 46.99) (end 38.83 46.99) (width 0.8) (layer F.Cu) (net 5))
 (segment (start 76.2 49.53) (end 74.3837 49.53) (width 0.8) (layer F.Cu) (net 3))
 (segment (start 66.2603 50.99) (end 64.26 50.99) (width 0.8) (layer F.Cu) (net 3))
 (segment (start 67.7203 49.53) (end 66.2603 50.99) (width 0.8) (layer F.Cu) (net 3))
 (segment (start 74.3837 49.53) (end 67.7203 49.53) (width 0.8) (layer F.Cu) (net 3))
 (segment (start 76.2 63.5097) (end 76.2 65.31) (width 0.8) (layer F.Cu) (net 3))
 (segment (start 76.5376 63.5097) (end 76.2 63.5097) (width 0.8) (layer F.Cu) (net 3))
 (segment (start 78.2728 61.7745) (end 76.5376 63.5097) (width 0.8) (layer F.Cu) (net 3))
 (segment (start 78.2728 56.42) (end 78.2728 61.7745) (width 0.8) (layer F.Cu) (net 3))
 (segment (start 79.2545 55.4383) (end 78.2728 56.42) (width 0.8) (layer F.Cu) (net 3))
 (segment (start 79.2545 47.0102) (end 79.2545 55.4383) (width 0.8) (layer F.Cu) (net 3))
 (segment (start 77.5703 45.326) (end 79.2545 47.0102) (width 0.8) (layer F.Cu) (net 3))
 (segment (start 74.7686 45.326) (end 77.5703 45.326) (width 0.8) (layer F.Cu) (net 3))
 (segment (start 74.3837 45.7109) (end 74.7686 45.326) (width 0.8) (layer F.Cu) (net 3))
 (segment (start 74.3837 49.53) (end 74.3837 45.7109) (width 0.8) (layer F.Cu) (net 3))
 (segment (start 78.2728 56.42) (end 76.2 56.42) (width 0.8) (layer F.Cu) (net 3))
 (segment (start 45.6883 48.99) (end 48.26 48.99) (width 0.8) (layer F.Cu) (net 15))
 (segment (start 40.7033 53.975) (end 45.6883 48.99) (width 0.8) (layer F.Cu) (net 15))
 (segment (start 40.005 53.975) (end 40.7033 53.975) (width 0.8) (layer F.Cu) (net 15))
 (segment (start 47.4443 60.325) (end 40.005 60.325) (width 0.8) (layer F.Cu) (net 10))
 (segment (start 47.8596 60.7403) (end 47.4443 60.325) (width 0.8) (layer F.Cu) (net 10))
 (segment (start 55.25 60.7403) (end 47.8596 60.7403) (width 0.8) (layer F.Cu) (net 10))
 (segment (start 55.25 58.74) (end 55.25 60.7403) (width 0.8) (layer F.Cu) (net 10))
 (segment (start 57.25 60.7403) (end 57.25 58.74) (width 0.8) (layer F.Cu) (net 11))
 (segment (start 56.0202 61.9701) (end 57.25 60.7403) (width 0.8) (layer F.Cu) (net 11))
 (segment (start 41.7519 61.9701) (end 56.0202 61.9701) (width 0.8) (layer F.Cu) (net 11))
 (segment (start 41.3768 61.595) (end 41.7519 61.9701) (width 0.8) (layer F.Cu) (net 11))
 (segment (start 40.005 61.595) (end 41.3768 61.595) (width 0.8) (layer F.Cu) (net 11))
 (segment (start 45.6318 50.99) (end 48.26 50.99) (width 0.8) (layer F.Cu) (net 16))
 (segment (start 41.3768 55.245) (end 45.6318 50.99) (width 0.8) (layer F.Cu) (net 16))
 (segment (start 40.005 55.245) (end 41.3768 55.245) (width 0.8) (layer F.Cu) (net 16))
 (segment (start 42.7347 56.515) (end 40.005 56.515) (width 0.8) (layer F.Cu) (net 17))
 (segment (start 46.2597 52.99) (end 42.7347 56.515) (width 0.8) (layer F.Cu) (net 17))
 (segment (start 48.26 52.99) (end 46.2597 52.99) (width 0.8) (layer F.Cu) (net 17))
 (segment (start 38.6332 57.785) (end 40.005 57.785) (width 0.8) (layer F.Cu) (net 17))
 (segment (start 38.6332 56.515) (end 38.6332 57.785) (width 0.8) (layer F.Cu) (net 17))
 (segment (start 40.005 56.515) (end 38.6332 56.515) (width 0.8) (layer F.Cu) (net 17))
 (segment (start 42.1947 59.055) (end 40.005 59.055) (width 0.8) (layer F.Cu) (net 18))
 (segment (start 46.2597 54.99) (end 42.1947 59.055) (width 0.8) (layer F.Cu) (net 18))
 (segment (start 48.26 54.99) (end 46.2597 54.99) (width 0.8) (layer F.Cu) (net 18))
 (segment (start 66.2603 52.99) (end 64.26 52.99) (width 0.8) (layer F.Cu) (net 7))
 (segment (start 67.7549 54.4846) (end 66.2603 52.99) (width 0.8) (layer F.Cu) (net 7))
 (segment (start 67.7549 57.7623) (end 67.7549 54.4846) (width 0.8) (layer F.Cu) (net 7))
 (segment (start 68.6123 58.6197) (end 67.7549 57.7623) (width 0.8) (layer F.Cu) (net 7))
 (segment (start 69.85 58.6197) (end 68.6123 58.6197) (width 0.8) (layer F.Cu) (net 7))
 (segment (start 69.85 60.42) (end 69.85 58.6197) (width 0.8) (layer F.Cu) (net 7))
 (segment (start 71.9047 62.4747) (end 69.85 60.42) (width 0.8) (layer F.Cu) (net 7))
 (segment (start 71.9047 70.7063) (end 71.9047 62.4747) (width 0.8) (layer F.Cu) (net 7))
 (segment (start 71.491 71.12) (end 71.9047 70.7063) (width 0.8) (layer F.Cu) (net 7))
 (segment (start 59.69 71.12) (end 71.491 71.12) (width 0.8) (layer F.Cu) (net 7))
 (segment (start 26.5682 46.99) (end 24.13 46.99) (width 0.8) (layer F.Cu) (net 23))
 (segment (start 32.2832 52.705) (end 26.5682 46.99) (width 0.8) (layer F.Cu) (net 23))
 (segment (start 33.655 52.705) (end 32.2832 52.705) (width 0.8) (layer F.Cu) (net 23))
 (segment (start 47.72 72.1377) (end 47.72 66.04) (width 0.8) (layer F.Cu) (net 23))
 (segment (start 44.4218 75.4359) (end 47.72 72.1377) (width 0.8) (layer F.Cu) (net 23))
 (segment (start 26.2526 75.4359) (end 44.4218 75.4359) (width 0.8) (layer F.Cu) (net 23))
 (segment (start 25.1249 74.3082) (end 26.2526 75.4359) (width 0.8) (layer F.Cu) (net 23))
 (segment (start 25.1249 72.7997) (end 25.1249 74.3082) (width 0.8) (layer F.Cu) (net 23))
 (segment (start 27.5537 70.3709) (end 25.1249 72.7997) (width 0.8) (layer F.Cu) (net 23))
 (segment (start 27.94 70.3709) (end 27.5537 70.3709) (width 0.8) (layer F.Cu) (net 23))
 (segment (start 27.94 68.58) (end 27.94 70.3709) (width 0.8) (layer F.Cu) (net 23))
 (segment (start 27.94 59.1437) (end 27.94 68.58) (width 0.8) (layer B.Cu) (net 23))
 (segment (start 25.9463 57.15) (end 27.94 59.1437) (width 0.8) (layer B.Cu) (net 23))
 (segment (start 24.13 57.15) (end 25.9463 57.15) (width 0.8) (layer B.Cu) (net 23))
 (segment (start 24.13 55.3337) (end 24.13 57.15) (width 0.8) (layer B.Cu) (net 23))
 (segment (start 22.3137 53.5174) (end 24.13 55.3337) (width 0.8) (layer B.Cu) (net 23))
 (segment (start 22.3137 46.99) (end 22.3137 53.5174) (width 0.8) (layer B.Cu) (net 23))
 (segment (start 24.13 46.99) (end 22.3137 46.99) (width 0.8) (layer B.Cu) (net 23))
 (segment (start 27.94 29.7309) (end 27.7776 29.7309) (width 0.8) (layer B.Cu) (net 23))
 (segment (start 24.13 33.216) (end 24.13 46.99) (width 0.8) (layer B.Cu) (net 23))
 (segment (start 27.6151 29.7309) (end 24.13 33.216) (width 0.8) (layer B.Cu) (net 23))
 (segment (start 27.7776 29.7309) (end 27.6151 29.7309) (width 0.8) (layer B.Cu) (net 23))
 (segment (start 27.94 29.8933) (end 27.94 30.48) (width 0.8) (layer B.Cu) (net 23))
 (segment (start 27.7776 29.7309) (end 27.94 29.8933) (width 0.8) (layer B.Cu) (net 23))
 (segment (start 31.9915 29.21) (end 40.64 29.21) (width 0.8) (layer F.Cu) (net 23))
 (segment (start 30.7215 30.48) (end 31.9915 29.21) (width 0.8) (layer F.Cu) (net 23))
 (segment (start 27.94 30.48) (end 30.7215 30.48) (width 0.8) (layer F.Cu) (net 23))
 (segment (start 45.72 66.2397) (end 45.72 71.12) (width 0.8) (layer F.Cu) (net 26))
 (segment (start 45.5203 66.04) (end 45.72 66.2397) (width 0.8) (layer F.Cu) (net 26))
 (segment (start 43.72 66.04) (end 45.5203 66.04) (width 0.8) (layer F.Cu) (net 26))
 (segment (start 35.0268 62.9668) (end 43.18 71.12) (width 0.8) (layer F.Cu) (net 27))
 (segment (start 35.0268 61.595) (end 35.0268 62.9668) (width 0.8) (layer F.Cu) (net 27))
 (segment (start 33.655 61.595) (end 35.0268 61.595) (width 0.8) (layer F.Cu) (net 27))
 (segment (start 32.2832 62.7632) (end 40.64 71.12) (width 0.8) (layer F.Cu) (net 28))
 (segment (start 32.2832 60.325) (end 32.2832 62.7632) (width 0.8) (layer F.Cu) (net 28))
 (segment (start 33.655 60.325) (end 32.2832 60.325) (width 0.8) (layer F.Cu) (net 28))
 (segment (start 31.8292 59.055) (end 33.655 59.055) (width 0.8) (layer F.Cu) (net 29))
 (segment (start 31.0677 59.8165) (end 31.8292 59.055) (width 0.8) (layer F.Cu) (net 29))
 (segment (start 31.0677 64.0542) (end 31.0677 59.8165) (width 0.8) (layer F.Cu) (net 29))
 (segment (start 36.4361 69.4226) (end 31.0677 64.0542) (width 0.8) (layer F.Cu) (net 29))
 (segment (start 36.4361 71.12) (end 36.4361 69.4226) (width 0.8) (layer F.Cu) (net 29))
 (segment (start 38.1 71.12) (end 36.4361 71.12) (width 0.8) (layer F.Cu) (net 29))
 (segment (start 32.2832 56.515) (end 32.2832 57.785) (width 0.8) (layer F.Cu) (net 31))
 (segment (start 33.655 56.515) (end 32.2832 56.515) (width 0.8) (layer F.Cu) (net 31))
 (segment (start 33.655 57.785) (end 32.2832 57.785) (width 0.8) (layer F.Cu) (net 31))
 (segment (start 31.3366 57.785) (end 32.2832 57.785) (width 0.8) (layer F.Cu) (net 31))
 (segment (start 29.8591 59.2625) (end 31.3366 57.785) (width 0.8) (layer F.Cu) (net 31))
 (segment (start 29.8591 65.3916) (end 29.8591 59.2625) (width 0.8) (layer F.Cu) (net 31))
 (segment (start 30.7454 66.2779) (end 29.8591 65.3916) (width 0.8) (layer F.Cu) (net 31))
 (segment (start 30.7454 69.3195) (end 30.7454 66.2779) (width 0.8) (layer F.Cu) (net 31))
 (segment (start 28.2758 71.7891) (end 30.7454 69.3195) (width 0.8) (layer F.Cu) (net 31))
 (segment (start 27.94 71.7891) (end 28.2758 71.7891) (width 0.8) (layer F.Cu) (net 31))
 (segment (start 27.94 73.58) (end 27.94 71.7891) (width 0.8) (layer F.Cu) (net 31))
 (segment (start 61.0006 30.48) (end 53.3019 30.48) (width 0.8) (layer F.Cu) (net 30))
 (segment (start 49.4919 34.29) (end 40.64 34.29) (width 0.8) (layer B.Cu) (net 30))
 (segment (start 53.3019 30.48) (end 49.4919 34.29) (width 0.8) (layer B.Cu) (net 30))
 (segment (start 30.3913 53.975) (end 33.655 53.975) (width 0.8) (layer F.Cu) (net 24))
 (segment (start 25.9463 49.53) (end 30.3913 53.975) (width 0.8) (layer F.Cu) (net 24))
 (segment (start 24.13 49.53) (end 25.9463 49.53) (width 0.8) (layer F.Cu) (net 24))
 (segment (start 26.7988 59.69) (end 24.13 59.69) (width 0.8) (layer F.Cu) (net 25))
 (segment (start 31.2438 55.245) (end 26.7988 59.69) (width 0.8) (layer F.Cu) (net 25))
 (segment (start 33.655 55.245) (end 31.2438 55.245) (width 0.8) (layer F.Cu) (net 25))
 (segment (start 78.0163 39.3087) (end 78.0163 35.56) (width 0.8) (layer F.Cu) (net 19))
 (segment (start 74.78 42.545) (end 78.0163 39.3087) (width 0.8) (layer F.Cu) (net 19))
 (segment (start 72.7053 42.545) (end 74.78 42.545) (width 0.8) (layer F.Cu) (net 19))
 (segment (start 66.2603 48.99) (end 72.7053 42.545) (width 0.8) (layer F.Cu) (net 19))
 (segment (start 64.26 48.99) (end 66.2603 48.99) (width 0.8) (layer F.Cu) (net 19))
 (segment (start 76.2 35.56) (end 78.0163 35.56) (width 0.8) (layer F.Cu) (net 19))
 (segment (start 78.0163 27.226) (end 78.0163 35.56) (width 0.8) (layer F.Cu) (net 19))
 (segment (start 77.4603 26.67) (end 78.0163 27.226) (width 0.8) (layer F.Cu) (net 19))
 (segment (start 75.66 26.67) (end 77.4603 26.67) (width 0.8) (layer F.Cu) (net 19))
 (segment (start 66.2603 46.99) (end 64.26 46.99) (width 0.8) (layer F.Cu) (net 20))
 (segment (start 66.2603 42.95) (end 66.2603 46.99) (width 0.8) (layer F.Cu) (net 20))
 (segment (start 71.12 38.0903) (end 66.2603 42.95) (width 0.8) (layer F.Cu) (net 20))
 (segment (start 71.12 36.29) (end 71.12 38.0903) (width 0.8) (layer F.Cu) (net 20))
 (segment (start 74.3837 33.02) (end 76.2 33.02) (width 0.8) (layer F.Cu) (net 20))
 (segment (start 72.914 34.4897) (end 74.3837 33.02) (width 0.8) (layer F.Cu) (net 20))
 (segment (start 71.12 34.4897) (end 72.914 34.4897) (width 0.8) (layer F.Cu) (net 20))
 (segment (start 71.12 36.29) (end 71.12 34.4897) (width 0.8) (layer F.Cu) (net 20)))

